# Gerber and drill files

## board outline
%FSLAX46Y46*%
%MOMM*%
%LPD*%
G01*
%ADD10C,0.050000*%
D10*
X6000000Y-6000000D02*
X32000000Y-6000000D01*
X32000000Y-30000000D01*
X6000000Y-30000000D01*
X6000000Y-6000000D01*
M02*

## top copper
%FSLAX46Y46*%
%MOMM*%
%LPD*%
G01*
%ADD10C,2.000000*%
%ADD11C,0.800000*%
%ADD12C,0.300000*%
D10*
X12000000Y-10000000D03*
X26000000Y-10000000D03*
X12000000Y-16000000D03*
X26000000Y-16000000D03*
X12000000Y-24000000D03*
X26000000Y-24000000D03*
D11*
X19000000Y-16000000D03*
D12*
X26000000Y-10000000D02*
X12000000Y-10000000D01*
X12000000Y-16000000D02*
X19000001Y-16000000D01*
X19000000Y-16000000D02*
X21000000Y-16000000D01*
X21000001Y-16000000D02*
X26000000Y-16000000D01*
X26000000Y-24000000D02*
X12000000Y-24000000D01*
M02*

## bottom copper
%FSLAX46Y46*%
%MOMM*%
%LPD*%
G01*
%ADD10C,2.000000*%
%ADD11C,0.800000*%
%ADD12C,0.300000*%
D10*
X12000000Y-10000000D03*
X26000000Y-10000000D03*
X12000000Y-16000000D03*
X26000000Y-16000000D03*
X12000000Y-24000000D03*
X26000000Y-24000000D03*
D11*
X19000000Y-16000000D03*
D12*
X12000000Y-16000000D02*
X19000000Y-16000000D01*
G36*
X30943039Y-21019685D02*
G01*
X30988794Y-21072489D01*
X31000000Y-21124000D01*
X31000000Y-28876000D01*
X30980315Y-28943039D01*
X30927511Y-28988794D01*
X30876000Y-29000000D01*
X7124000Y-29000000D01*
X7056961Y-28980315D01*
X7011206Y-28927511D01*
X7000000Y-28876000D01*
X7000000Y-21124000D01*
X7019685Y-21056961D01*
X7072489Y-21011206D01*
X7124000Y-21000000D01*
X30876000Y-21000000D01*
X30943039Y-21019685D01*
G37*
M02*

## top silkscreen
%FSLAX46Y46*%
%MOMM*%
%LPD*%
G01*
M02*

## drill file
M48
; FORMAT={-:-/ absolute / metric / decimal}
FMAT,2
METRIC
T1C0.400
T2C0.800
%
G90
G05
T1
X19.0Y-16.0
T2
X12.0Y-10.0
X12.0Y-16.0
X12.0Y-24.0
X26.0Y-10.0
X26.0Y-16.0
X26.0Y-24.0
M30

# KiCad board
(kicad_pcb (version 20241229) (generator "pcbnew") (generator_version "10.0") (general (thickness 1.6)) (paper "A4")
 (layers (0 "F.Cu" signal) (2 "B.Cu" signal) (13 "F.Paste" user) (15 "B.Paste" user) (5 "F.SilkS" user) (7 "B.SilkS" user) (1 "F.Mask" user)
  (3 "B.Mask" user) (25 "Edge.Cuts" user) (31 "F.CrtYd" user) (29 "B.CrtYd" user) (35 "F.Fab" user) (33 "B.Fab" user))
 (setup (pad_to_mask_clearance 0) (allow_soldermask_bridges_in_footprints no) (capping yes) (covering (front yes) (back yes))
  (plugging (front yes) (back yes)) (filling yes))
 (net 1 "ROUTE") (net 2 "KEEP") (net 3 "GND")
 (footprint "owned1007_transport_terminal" (layer "F.Cu") (at 12 10)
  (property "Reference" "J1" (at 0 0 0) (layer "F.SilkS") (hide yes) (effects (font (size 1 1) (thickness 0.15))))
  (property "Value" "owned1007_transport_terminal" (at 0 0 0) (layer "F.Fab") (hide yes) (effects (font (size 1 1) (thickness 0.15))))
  (pad "1" thru_hole circle (at 0 0) (size 2 2) (drill 0.8) (layers "*.Cu" "*.Mask") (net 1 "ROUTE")))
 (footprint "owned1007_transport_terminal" (layer "F.Cu") (at 26 10)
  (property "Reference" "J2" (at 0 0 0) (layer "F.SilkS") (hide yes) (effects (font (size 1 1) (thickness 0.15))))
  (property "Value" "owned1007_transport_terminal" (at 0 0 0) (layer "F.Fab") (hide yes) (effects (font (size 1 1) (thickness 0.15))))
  (pad "1" thru_hole circle (at 0 0) (size 2 2) (drill 0.8) (layers "*.Cu" "*.Mask") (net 1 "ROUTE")))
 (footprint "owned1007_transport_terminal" (layer "F.Cu") (at 12 16)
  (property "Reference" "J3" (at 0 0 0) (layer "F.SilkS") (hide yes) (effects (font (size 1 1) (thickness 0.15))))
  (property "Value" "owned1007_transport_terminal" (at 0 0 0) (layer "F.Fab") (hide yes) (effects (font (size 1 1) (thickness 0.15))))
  (pad "1" thru_hole circle (at 0 0) (size 2 2) (drill 0.8) (layers "*.Cu" "*.Mask") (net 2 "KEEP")))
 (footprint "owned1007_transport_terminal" (layer "F.Cu") (at 26 16)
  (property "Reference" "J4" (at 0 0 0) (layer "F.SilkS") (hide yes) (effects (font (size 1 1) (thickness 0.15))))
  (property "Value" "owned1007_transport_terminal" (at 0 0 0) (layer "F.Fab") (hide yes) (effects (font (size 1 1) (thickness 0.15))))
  (pad "1" thru_hole circle (at 0 0) (size 2 2) (drill 0.8) (layers "*.Cu" "*.Mask") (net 2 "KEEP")))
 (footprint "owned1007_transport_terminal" (layer "F.Cu") (at 12 24)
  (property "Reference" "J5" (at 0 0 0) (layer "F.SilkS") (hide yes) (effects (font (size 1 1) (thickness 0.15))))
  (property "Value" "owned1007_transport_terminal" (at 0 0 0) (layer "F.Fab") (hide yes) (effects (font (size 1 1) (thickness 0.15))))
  (pad "1" thru_hole circle (at 0 0) (size 2 2) (drill 0.8) (layers "*.Cu" "*.Mask") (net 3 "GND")))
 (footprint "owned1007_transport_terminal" (layer "F.Cu") (at 26 24)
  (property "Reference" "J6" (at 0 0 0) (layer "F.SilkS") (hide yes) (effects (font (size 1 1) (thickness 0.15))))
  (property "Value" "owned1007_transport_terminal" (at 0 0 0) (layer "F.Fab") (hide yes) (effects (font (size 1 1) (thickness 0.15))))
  (pad "1" thru_hole circle (at 0 0) (size 2 2) (drill 0.8) (layers "*.Cu" "*.Mask") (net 3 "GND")))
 (gr_rect (start 6 6) (end 32 30) (stroke (width 0.05) (type default)) (fill none) (layer "Edge.Cuts"))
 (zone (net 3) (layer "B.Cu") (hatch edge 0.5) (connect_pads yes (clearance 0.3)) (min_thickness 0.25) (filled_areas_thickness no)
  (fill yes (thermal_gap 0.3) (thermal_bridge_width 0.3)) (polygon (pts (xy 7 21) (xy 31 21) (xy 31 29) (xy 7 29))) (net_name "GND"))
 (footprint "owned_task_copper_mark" (layer "F.Cu") (at 10 28)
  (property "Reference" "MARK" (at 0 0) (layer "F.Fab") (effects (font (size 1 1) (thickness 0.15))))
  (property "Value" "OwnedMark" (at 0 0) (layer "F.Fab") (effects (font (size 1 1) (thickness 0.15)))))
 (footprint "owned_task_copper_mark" (layer "F.Cu") (at 13 28)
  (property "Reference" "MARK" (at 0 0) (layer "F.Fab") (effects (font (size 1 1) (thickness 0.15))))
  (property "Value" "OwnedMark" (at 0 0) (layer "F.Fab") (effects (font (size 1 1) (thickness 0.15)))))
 (segment (start 26 10) (end 12 10) (width 0.3) (layer "F.Cu") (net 1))
 (segment (start 12 16) (end 19.000001 16) (width 0.3) (layer "F.Cu") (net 2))
 (segment (start 19 16) (end 21 16) (width 0.3) (layer "F.Cu") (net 2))
 (segment (start 21.000001 16) (end 26 16) (width 0.3) (layer "F.Cu") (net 2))
 (via (at 19 16) (size 0.8) (drill 0.4) (layers "F.Cu" "B.Cu") (free yes) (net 2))
 (segment (start 12 16) (end 19 16) (width 0.3) (layer "B.Cu") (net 2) (locked yes))
 (segment (start 26 24) (end 12 24) (width 0.3) (layer "F.Cu") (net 3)))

